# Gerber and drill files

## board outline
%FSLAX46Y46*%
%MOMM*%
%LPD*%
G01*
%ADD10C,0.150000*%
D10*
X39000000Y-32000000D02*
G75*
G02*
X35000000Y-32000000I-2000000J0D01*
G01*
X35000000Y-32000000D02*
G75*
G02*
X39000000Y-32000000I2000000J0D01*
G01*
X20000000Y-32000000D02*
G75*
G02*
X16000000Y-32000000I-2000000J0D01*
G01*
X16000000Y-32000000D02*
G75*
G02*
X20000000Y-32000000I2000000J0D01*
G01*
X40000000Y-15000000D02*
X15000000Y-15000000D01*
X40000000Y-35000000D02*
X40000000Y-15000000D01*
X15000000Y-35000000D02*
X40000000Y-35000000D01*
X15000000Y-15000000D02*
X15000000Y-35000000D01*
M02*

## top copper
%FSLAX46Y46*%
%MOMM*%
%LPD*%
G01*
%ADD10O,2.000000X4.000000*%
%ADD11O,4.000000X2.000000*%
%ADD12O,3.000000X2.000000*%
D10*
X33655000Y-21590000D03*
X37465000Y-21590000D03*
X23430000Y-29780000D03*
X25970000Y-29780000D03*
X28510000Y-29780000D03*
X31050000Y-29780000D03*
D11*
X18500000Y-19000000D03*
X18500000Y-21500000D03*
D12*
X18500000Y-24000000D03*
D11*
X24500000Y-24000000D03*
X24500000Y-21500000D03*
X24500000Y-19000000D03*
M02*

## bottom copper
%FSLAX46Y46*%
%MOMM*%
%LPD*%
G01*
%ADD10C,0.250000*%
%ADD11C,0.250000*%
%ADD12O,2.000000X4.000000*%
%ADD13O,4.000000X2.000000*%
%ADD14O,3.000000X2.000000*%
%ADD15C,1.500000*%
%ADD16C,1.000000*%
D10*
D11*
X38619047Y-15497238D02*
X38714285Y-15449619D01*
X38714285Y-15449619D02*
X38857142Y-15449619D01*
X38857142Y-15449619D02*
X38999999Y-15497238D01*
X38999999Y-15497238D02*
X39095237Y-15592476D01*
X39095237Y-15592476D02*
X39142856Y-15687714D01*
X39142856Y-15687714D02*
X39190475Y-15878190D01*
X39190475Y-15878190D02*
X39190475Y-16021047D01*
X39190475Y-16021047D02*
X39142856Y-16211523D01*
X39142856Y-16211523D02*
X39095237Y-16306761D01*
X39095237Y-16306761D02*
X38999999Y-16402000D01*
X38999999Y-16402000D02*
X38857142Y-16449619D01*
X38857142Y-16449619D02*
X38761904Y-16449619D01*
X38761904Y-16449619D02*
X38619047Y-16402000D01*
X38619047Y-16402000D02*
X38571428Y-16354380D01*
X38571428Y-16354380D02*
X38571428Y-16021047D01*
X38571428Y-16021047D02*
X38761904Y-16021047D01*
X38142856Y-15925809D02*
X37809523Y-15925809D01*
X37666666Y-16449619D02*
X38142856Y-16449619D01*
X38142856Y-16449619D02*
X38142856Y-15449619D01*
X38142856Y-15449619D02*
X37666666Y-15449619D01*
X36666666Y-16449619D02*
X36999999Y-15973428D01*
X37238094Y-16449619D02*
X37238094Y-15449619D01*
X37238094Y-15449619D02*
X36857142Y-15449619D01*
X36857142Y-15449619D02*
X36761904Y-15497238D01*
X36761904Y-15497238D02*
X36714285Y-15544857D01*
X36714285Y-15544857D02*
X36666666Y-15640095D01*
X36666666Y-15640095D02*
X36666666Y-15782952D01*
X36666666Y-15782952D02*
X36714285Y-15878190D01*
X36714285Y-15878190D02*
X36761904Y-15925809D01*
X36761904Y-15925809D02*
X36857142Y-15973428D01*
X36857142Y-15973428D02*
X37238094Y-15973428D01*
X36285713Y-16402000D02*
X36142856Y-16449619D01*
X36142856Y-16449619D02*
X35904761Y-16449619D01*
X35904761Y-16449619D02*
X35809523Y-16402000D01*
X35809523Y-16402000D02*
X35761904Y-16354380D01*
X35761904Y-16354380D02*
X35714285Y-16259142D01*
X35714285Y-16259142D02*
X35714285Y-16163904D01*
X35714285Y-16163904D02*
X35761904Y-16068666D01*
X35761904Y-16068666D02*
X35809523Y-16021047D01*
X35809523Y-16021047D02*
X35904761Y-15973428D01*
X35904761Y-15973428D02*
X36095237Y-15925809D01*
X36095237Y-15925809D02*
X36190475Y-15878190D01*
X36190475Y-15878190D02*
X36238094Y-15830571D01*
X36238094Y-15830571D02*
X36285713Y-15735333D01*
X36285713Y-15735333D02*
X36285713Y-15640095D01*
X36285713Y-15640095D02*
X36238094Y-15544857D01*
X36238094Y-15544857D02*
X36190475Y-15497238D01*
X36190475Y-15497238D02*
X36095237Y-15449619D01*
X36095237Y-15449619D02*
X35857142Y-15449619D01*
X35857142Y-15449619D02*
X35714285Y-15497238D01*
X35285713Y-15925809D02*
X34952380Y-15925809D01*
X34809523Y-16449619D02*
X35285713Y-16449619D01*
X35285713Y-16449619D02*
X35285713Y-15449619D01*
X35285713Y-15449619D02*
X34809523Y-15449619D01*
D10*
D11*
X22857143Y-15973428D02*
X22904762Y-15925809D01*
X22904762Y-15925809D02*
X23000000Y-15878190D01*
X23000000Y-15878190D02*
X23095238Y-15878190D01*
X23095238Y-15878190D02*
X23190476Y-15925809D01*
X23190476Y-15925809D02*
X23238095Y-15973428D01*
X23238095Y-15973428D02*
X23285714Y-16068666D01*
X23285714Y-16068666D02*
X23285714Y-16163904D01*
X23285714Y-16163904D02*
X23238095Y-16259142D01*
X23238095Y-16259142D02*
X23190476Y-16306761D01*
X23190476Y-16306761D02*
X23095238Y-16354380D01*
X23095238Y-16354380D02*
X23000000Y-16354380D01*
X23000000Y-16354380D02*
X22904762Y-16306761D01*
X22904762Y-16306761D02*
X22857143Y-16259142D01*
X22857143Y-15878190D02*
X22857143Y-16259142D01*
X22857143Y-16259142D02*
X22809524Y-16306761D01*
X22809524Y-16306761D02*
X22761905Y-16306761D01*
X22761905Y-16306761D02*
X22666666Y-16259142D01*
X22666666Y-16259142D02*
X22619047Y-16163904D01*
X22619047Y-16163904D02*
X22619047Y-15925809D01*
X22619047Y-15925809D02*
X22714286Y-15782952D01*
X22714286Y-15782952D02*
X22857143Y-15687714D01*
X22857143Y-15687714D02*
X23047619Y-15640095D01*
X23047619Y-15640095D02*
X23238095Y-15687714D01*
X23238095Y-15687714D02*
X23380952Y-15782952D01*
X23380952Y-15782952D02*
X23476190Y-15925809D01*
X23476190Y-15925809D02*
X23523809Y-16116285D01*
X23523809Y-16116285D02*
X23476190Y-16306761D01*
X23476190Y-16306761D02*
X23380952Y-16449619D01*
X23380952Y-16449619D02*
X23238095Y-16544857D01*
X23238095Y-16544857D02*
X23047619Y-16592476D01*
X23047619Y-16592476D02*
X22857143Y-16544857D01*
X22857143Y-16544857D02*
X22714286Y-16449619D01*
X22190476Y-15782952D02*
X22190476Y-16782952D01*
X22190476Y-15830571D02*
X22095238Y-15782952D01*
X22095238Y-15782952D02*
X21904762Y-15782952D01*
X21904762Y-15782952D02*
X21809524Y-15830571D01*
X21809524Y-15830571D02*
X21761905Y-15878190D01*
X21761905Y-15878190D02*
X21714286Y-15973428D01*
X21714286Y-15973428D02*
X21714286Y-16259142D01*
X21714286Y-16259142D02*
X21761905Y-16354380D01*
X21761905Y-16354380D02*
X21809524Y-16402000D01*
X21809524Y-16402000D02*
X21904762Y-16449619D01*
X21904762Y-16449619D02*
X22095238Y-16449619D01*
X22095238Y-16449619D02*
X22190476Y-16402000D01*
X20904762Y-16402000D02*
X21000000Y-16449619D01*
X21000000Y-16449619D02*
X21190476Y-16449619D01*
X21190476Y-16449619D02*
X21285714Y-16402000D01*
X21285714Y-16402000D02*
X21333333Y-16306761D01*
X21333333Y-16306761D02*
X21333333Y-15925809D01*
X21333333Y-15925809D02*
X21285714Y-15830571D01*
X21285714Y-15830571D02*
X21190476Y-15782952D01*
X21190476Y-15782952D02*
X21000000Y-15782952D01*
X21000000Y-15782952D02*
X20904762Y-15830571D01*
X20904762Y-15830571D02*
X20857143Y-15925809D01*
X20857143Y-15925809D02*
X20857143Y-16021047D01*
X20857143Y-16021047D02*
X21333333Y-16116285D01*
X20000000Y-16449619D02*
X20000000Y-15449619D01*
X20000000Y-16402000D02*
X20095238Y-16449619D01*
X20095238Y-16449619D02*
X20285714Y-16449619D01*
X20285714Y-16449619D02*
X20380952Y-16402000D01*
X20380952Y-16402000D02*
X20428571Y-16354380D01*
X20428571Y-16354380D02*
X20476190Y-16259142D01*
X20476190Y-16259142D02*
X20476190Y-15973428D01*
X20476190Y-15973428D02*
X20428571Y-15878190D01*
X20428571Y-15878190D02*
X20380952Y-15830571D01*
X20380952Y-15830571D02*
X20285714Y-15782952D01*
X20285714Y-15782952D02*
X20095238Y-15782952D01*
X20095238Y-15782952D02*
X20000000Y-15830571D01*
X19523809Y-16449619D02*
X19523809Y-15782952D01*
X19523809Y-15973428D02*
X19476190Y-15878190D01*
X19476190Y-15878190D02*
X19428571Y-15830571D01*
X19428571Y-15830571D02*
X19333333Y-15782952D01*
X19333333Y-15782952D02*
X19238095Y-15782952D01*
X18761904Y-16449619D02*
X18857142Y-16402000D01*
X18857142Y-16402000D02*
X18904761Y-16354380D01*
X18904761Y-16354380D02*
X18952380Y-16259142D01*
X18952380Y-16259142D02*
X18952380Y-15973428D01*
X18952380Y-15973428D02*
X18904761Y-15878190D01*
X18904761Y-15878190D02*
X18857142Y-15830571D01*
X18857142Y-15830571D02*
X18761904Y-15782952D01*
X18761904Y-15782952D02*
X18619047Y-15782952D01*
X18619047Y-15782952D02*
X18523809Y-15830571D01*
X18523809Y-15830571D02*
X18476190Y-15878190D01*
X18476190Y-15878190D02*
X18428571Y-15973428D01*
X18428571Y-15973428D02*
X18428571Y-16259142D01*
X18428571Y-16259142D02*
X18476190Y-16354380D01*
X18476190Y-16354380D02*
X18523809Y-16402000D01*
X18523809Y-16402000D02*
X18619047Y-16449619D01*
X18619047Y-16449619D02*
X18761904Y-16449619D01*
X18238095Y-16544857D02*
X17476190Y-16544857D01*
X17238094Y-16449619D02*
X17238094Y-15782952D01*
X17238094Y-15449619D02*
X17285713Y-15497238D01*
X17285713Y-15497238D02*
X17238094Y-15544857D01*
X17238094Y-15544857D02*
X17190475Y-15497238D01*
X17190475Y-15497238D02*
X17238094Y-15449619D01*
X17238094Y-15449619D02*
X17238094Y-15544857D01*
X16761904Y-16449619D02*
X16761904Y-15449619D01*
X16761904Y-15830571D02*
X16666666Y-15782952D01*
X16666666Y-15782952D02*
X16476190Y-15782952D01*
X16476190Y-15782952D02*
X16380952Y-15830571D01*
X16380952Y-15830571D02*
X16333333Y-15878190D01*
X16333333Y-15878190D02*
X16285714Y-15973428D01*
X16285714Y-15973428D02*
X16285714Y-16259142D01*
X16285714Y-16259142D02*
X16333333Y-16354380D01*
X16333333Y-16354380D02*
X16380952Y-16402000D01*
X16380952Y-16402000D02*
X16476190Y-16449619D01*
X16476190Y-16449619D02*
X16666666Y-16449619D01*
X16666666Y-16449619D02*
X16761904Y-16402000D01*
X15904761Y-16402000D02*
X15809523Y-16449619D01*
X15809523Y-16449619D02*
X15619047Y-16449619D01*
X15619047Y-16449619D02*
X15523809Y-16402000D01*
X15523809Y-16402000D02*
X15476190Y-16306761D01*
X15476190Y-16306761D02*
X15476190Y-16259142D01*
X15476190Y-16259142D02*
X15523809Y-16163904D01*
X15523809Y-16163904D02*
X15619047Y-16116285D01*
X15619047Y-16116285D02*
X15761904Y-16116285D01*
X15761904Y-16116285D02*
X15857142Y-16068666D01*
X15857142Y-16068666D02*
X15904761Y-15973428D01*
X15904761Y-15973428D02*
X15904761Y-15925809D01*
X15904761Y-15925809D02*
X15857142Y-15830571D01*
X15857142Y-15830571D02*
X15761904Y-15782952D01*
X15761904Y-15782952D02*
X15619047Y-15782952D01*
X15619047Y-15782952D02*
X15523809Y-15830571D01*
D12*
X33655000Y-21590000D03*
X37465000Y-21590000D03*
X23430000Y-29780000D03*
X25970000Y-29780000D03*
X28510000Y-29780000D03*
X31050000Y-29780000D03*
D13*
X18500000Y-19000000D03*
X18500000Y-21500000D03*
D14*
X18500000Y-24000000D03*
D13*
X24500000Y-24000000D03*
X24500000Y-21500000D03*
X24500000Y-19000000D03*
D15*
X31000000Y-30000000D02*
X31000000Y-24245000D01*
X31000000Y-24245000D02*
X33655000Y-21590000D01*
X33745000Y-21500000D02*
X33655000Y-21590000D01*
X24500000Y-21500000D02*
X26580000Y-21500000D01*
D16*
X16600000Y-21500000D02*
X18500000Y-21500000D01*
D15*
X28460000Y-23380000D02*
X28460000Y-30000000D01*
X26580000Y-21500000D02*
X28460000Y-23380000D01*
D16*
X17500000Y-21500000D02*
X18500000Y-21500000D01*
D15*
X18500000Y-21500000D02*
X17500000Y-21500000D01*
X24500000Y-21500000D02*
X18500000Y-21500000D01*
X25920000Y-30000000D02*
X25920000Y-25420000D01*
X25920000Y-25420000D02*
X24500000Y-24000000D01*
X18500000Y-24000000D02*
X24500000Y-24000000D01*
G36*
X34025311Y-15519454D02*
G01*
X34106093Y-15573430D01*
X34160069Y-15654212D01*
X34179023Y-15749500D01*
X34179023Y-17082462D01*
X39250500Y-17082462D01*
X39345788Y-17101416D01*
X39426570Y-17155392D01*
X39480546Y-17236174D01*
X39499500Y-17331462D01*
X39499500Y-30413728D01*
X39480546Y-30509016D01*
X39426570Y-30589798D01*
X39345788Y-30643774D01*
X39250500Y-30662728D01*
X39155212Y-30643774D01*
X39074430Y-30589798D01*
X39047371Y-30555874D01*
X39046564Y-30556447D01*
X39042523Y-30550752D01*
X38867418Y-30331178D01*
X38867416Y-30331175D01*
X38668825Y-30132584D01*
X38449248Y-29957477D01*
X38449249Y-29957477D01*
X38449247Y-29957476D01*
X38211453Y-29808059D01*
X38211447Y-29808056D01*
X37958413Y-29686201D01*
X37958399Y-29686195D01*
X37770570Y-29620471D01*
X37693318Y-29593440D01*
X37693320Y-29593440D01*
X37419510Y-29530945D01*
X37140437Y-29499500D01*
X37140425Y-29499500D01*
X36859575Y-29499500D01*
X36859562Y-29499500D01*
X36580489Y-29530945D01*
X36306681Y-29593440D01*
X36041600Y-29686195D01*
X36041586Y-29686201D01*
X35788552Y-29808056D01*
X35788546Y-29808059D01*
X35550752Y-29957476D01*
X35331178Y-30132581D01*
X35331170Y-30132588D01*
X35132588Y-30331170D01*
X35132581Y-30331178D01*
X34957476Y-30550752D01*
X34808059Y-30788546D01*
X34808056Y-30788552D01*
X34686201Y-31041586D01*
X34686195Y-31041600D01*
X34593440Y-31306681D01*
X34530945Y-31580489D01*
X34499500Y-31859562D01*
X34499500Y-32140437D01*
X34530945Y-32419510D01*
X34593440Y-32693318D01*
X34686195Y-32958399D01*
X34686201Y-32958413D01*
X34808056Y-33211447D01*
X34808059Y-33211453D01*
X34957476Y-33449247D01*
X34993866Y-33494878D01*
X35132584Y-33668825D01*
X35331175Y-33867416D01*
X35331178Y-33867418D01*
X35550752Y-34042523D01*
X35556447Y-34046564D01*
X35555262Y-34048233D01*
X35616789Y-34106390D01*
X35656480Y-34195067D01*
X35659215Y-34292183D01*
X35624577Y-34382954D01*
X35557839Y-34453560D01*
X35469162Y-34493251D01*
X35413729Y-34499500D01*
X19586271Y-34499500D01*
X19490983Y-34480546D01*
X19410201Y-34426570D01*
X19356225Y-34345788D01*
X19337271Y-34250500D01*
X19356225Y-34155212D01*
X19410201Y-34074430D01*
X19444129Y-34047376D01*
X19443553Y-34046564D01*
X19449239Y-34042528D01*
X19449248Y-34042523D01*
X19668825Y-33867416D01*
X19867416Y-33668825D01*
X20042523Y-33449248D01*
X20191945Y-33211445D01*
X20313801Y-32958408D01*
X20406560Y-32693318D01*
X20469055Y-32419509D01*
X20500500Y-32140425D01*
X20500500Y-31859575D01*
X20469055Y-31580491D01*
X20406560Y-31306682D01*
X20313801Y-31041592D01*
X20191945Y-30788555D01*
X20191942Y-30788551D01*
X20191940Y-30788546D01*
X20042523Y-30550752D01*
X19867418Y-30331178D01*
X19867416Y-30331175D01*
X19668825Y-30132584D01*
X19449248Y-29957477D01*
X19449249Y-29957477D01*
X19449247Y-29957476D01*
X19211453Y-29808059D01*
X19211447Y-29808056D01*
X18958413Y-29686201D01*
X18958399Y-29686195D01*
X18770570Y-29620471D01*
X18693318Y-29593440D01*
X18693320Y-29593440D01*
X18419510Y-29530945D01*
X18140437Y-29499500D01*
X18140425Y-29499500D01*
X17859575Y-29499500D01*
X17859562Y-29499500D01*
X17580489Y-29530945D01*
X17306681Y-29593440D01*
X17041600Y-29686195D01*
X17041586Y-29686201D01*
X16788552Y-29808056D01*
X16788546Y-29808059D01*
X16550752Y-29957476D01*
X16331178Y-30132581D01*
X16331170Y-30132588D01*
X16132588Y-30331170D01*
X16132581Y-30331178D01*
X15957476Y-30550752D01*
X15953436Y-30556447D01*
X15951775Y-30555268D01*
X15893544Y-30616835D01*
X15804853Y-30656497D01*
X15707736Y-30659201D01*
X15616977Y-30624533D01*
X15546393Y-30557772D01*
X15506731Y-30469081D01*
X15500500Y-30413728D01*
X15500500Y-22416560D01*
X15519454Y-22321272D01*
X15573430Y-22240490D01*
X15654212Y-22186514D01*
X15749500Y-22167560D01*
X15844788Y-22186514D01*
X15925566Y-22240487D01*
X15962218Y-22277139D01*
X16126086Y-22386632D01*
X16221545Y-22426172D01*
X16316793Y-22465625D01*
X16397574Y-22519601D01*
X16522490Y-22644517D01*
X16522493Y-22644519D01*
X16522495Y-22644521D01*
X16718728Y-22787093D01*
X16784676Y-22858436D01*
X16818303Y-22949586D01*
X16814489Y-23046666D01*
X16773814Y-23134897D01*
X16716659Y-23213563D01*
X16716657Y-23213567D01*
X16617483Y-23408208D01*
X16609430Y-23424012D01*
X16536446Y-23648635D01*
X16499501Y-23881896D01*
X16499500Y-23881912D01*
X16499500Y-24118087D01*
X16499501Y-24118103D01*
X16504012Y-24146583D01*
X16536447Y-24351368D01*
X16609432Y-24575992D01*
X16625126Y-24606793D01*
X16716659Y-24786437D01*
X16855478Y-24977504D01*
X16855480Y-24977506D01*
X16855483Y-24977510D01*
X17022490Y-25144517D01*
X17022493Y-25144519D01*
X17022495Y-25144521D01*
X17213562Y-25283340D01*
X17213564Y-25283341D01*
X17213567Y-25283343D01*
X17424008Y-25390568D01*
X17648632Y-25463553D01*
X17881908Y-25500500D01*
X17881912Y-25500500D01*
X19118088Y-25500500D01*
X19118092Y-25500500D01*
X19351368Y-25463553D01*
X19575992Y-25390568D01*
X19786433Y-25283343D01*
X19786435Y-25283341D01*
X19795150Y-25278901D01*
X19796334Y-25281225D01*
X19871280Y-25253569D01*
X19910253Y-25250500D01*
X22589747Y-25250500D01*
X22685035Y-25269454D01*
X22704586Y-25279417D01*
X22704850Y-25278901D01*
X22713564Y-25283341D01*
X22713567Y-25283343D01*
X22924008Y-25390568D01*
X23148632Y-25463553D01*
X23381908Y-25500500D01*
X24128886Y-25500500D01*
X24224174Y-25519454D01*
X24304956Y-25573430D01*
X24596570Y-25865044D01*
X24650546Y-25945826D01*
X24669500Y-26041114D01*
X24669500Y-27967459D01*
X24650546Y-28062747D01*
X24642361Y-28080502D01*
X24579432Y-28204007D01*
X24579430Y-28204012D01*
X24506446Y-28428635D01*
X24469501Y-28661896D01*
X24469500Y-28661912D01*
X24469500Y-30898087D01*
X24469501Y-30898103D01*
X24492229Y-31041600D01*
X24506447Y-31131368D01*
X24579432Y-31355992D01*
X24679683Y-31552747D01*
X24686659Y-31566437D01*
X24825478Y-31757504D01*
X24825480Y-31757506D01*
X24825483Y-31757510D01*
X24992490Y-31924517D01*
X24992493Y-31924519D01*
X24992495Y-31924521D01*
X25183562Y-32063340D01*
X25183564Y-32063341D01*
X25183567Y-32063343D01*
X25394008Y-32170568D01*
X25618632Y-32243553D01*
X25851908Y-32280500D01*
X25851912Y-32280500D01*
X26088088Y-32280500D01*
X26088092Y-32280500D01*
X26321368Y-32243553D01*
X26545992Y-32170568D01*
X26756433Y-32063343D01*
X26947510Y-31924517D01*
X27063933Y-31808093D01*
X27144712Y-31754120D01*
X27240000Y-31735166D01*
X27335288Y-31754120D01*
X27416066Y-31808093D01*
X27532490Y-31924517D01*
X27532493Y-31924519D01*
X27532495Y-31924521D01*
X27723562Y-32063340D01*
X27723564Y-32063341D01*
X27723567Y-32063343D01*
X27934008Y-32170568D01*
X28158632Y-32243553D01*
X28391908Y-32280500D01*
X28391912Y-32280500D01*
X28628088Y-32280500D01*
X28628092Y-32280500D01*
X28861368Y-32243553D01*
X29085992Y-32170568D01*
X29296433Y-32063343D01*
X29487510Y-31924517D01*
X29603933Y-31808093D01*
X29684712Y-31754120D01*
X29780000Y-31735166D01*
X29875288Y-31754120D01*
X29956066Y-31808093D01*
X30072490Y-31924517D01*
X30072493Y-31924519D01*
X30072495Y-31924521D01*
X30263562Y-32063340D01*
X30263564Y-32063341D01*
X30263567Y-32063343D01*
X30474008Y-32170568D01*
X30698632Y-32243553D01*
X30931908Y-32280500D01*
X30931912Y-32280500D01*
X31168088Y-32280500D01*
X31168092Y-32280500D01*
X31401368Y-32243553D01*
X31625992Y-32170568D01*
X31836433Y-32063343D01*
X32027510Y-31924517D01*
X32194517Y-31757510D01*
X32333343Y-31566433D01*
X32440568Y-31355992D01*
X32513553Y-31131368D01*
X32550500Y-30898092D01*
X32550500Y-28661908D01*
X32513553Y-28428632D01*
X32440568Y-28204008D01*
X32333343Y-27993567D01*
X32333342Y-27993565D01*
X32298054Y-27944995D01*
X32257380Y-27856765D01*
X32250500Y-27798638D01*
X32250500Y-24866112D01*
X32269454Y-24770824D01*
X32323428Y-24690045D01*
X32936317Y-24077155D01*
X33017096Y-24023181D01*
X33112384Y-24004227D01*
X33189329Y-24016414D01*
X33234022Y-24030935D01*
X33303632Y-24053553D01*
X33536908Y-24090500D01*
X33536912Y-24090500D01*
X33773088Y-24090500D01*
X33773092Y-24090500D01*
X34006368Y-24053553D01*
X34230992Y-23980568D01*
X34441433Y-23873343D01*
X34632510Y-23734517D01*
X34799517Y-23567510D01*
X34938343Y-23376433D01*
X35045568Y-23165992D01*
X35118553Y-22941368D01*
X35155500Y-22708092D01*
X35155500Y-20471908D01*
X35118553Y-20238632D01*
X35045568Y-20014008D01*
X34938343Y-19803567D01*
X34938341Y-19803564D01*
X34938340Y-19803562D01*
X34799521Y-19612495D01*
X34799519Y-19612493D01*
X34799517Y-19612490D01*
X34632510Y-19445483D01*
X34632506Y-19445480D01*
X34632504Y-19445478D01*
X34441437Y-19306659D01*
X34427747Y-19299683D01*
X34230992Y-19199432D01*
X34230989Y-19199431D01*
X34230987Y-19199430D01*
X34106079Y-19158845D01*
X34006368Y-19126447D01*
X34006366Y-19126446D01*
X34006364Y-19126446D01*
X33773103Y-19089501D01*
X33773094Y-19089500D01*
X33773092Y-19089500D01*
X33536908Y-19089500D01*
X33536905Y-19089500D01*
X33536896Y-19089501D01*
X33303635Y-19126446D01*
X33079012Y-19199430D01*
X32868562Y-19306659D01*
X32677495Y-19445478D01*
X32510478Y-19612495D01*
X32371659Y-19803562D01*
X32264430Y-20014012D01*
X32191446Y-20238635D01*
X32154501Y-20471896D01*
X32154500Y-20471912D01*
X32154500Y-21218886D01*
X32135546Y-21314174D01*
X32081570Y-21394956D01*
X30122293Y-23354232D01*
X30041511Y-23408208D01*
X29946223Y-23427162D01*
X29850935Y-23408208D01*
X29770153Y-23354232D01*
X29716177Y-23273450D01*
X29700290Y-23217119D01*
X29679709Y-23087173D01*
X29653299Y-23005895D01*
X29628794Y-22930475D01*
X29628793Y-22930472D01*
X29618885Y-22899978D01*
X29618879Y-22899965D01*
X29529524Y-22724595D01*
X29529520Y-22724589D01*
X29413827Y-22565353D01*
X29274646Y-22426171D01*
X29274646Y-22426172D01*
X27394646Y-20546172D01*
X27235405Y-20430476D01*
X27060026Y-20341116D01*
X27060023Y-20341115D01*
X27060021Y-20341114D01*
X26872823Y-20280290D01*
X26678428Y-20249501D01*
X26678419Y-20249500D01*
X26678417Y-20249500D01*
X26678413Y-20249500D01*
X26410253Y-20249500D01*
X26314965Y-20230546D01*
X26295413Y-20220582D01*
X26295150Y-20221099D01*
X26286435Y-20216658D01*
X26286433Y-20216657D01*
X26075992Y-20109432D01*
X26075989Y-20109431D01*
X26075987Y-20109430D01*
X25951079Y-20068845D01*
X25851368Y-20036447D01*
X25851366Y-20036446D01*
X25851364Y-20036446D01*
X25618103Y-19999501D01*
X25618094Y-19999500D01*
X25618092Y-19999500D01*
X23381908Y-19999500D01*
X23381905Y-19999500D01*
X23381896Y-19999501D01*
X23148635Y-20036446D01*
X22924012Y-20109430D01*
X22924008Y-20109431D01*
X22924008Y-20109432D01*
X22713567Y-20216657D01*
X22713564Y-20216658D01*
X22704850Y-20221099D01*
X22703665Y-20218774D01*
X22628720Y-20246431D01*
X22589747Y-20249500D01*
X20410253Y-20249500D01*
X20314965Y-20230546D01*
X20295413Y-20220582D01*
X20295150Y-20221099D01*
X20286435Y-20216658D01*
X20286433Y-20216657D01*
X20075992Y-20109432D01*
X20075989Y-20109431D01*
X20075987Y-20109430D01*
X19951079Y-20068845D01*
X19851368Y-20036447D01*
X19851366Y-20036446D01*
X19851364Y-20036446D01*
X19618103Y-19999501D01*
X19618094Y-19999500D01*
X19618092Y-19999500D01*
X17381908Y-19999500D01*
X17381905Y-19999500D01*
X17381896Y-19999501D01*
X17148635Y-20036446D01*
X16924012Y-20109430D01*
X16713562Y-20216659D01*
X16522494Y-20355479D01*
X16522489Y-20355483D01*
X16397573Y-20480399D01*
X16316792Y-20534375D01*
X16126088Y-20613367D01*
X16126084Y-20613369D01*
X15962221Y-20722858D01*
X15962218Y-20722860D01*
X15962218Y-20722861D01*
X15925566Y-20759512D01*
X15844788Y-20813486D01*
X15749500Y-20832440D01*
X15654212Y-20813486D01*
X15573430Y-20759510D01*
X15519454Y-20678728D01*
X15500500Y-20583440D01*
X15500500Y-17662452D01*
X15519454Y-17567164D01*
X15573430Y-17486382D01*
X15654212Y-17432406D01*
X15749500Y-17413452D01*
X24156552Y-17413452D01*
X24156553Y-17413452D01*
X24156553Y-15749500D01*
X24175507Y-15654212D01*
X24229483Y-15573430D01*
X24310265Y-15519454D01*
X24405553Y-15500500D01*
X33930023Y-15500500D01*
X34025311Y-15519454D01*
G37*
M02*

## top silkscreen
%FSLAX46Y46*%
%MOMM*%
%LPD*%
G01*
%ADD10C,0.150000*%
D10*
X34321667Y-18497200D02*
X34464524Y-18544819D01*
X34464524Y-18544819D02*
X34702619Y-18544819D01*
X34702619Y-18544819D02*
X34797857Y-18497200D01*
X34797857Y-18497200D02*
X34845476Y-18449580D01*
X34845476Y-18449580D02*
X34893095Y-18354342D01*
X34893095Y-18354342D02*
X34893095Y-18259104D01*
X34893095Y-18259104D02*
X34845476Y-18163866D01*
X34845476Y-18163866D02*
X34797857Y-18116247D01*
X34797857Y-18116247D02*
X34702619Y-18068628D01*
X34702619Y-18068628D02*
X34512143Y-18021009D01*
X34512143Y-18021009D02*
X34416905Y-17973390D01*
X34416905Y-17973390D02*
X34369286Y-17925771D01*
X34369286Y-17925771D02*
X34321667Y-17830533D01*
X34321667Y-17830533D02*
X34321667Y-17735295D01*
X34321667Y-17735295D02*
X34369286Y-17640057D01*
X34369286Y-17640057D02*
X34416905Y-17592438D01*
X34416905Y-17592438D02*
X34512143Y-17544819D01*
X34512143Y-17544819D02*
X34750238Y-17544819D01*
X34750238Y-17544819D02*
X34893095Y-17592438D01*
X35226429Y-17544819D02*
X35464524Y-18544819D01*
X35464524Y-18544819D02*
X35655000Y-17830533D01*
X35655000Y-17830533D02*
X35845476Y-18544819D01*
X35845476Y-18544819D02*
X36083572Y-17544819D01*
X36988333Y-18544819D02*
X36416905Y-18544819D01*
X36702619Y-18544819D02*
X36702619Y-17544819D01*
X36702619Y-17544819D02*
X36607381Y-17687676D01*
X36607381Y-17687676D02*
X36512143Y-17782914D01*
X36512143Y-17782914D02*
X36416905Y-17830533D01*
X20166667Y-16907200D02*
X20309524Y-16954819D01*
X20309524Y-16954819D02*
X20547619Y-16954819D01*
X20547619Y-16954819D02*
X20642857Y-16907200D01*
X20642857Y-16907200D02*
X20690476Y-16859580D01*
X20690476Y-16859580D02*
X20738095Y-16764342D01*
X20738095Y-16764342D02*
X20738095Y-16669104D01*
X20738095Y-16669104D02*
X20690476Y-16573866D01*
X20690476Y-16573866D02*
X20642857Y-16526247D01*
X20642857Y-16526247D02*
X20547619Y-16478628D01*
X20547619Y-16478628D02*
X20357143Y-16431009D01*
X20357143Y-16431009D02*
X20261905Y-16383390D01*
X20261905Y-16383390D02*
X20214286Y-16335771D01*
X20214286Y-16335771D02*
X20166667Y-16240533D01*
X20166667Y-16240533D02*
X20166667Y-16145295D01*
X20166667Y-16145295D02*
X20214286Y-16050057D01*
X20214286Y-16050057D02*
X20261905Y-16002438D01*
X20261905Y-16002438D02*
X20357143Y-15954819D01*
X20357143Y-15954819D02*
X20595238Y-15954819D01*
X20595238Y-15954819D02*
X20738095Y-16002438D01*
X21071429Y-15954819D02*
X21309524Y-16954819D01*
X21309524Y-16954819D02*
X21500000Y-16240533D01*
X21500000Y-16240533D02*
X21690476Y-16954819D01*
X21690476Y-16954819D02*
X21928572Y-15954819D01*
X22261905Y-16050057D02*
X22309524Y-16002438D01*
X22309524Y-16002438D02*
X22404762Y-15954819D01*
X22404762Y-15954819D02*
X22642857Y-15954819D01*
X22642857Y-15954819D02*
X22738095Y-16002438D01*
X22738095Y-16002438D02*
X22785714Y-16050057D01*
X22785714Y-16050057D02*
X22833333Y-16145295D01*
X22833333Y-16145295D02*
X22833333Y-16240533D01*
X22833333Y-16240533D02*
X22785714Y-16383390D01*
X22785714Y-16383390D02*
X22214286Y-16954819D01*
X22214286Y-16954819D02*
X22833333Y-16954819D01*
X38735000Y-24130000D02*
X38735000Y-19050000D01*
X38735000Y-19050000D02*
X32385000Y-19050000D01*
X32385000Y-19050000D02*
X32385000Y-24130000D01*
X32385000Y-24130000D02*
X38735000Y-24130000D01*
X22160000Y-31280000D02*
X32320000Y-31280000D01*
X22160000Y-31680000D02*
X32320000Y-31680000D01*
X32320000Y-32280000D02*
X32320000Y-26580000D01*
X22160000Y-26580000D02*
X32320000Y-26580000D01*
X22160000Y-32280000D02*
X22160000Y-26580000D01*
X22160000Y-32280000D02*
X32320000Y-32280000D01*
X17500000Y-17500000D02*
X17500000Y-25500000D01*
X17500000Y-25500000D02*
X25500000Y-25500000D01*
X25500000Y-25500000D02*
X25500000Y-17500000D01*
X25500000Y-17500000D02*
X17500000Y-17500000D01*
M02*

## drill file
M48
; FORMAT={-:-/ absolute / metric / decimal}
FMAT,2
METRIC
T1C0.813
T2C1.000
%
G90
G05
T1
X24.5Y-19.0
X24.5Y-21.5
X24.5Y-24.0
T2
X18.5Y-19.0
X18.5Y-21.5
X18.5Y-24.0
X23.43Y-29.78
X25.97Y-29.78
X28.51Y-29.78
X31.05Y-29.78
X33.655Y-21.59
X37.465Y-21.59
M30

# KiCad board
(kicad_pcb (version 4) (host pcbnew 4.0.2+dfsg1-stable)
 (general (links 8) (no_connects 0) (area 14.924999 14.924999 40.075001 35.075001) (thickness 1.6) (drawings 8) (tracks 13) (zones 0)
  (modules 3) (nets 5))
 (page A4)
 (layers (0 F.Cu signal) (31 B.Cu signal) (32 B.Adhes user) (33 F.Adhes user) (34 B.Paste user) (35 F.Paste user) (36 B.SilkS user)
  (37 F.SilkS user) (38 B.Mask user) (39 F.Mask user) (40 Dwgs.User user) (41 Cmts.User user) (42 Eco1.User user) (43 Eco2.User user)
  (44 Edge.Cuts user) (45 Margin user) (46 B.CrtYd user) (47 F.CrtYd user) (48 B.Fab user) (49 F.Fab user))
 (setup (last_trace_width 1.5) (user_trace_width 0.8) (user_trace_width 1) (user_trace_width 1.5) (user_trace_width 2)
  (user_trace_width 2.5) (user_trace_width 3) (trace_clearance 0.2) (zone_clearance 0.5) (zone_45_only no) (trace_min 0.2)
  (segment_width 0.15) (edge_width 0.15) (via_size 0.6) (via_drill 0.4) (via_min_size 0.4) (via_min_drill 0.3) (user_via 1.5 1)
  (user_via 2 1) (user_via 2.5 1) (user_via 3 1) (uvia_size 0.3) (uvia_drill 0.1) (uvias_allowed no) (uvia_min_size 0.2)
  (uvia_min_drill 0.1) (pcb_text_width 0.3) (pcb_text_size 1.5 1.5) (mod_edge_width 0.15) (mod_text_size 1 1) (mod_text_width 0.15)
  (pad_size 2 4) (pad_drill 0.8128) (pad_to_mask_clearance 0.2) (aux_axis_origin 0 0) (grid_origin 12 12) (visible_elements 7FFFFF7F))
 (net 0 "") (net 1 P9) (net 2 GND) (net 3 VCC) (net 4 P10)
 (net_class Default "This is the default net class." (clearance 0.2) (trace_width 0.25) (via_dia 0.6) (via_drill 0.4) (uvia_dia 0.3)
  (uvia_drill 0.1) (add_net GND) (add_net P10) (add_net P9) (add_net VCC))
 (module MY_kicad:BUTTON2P (layer F.Cu) (at 33.655 21.59)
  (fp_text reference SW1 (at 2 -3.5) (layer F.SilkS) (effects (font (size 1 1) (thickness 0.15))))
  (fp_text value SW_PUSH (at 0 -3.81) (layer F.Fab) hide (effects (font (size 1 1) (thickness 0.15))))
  (fp_line (start 5.08 2.54) (end 5.08 -2.54) (layer F.SilkS) (width 0.15))
  (fp_line (start 5.08 -2.54) (end -1.27 -2.54) (layer F.SilkS) (width 0.15))
  (fp_line (start -1.27 -2.54) (end -1.27 2.54) (layer F.SilkS) (width 0.15))
  (fp_line (start -1.27 2.54) (end 5.08 2.54) (layer F.SilkS) (width 0.15))
  (pad 1 thru_hole oval (at 0 0) (size 2 4) (drill 1) (layers *.Cu *.Mask) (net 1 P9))
  (pad 2 thru_hole oval (at 3.81 0) (size 2 4) (drill 1) (layers *.Cu *.Mask) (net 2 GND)))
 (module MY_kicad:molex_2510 (layer F.Cu) (at 23.43 29.78)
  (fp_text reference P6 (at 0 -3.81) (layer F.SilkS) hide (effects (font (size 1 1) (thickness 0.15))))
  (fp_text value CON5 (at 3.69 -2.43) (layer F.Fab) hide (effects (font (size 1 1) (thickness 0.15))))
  (fp_line (start -1.27 1.5) (end 8.89 1.5) (layer F.SilkS) (width 0.15))
  (fp_line (start -1.27 1.9) (end 8.89 1.9) (layer F.SilkS) (width 0.15))
  (fp_line (start 8.89 2.5) (end 8.89 -3.2) (layer F.SilkS) (width 0.15))
  (fp_line (start -1.27 -3.2) (end 8.89 -3.2) (layer F.SilkS) (width 0.15))
  (fp_line (start -1.27 2.5) (end -1.27 -3.2) (layer F.SilkS) (width 0.15))
  (fp_line (start -1.27 2.5) (end 8.89 2.5) (layer F.SilkS) (width 0.15))
  (pad 1 thru_hole oval (at 0 0) (size 2 4) (drill 1) (layers *.Cu *.Mask) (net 2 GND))
  (pad 2 thru_hole oval (at 2.54 0) (size 2 4) (drill 1) (layers *.Cu *.Mask) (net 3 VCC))
  (pad 3 thru_hole oval (at 5.08 0) (size 2 4) (drill 1) (layers *.Cu *.Mask) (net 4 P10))
  (pad 4 thru_hole oval (at 7.62 0) (size 2 4) (drill 1) (layers *.Cu *.Mask) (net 1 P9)))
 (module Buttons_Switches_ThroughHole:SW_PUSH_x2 (layer F.Cu) (at 18.5 19 270)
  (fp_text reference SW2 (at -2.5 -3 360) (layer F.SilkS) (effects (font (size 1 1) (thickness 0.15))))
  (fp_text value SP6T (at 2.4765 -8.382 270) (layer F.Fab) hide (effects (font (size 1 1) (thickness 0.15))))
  (fp_line (start -1.5 1) (end 6.5 1) (layer F.SilkS) (width 0.15))
  (fp_line (start 6.5 1) (end 6.5 -7) (layer F.SilkS) (width 0.15))
  (fp_line (start 6.5 -7) (end -1.5 -7) (layer F.SilkS) (width 0.15))
  (fp_line (start -1.5 -7) (end -1.5 1) (layer F.SilkS) (width 0.15))
  (pad 1 thru_hole oval (at 0 0 270) (size 2 4) (drill 1) (layers *.Cu *.Mask) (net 2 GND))
  (pad 2 thru_hole oval (at 2.5 0 270) (size 2 4) (drill 1) (layers *.Cu B.Mask) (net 4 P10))
  (pad 3 thru_hole oval (at 5 0 270) (size 2 3) (drill 1) (layers *.Cu *.Mask) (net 3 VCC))
  (pad 4 thru_hole oval (at 5 -6 270) (size 2 4) (drill 0.8128) (layers *.Cu *.Mask) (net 3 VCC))
  (pad 5 thru_hole oval (at 2.5 -6 270) (size 2 4) (drill 0.8128) (layers *.Cu *.Mask) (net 4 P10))
  (pad 6 thru_hole oval (at 0 -6 270) (size 2 4) (drill 0.8128) (layers *.Cu *.Mask) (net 2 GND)))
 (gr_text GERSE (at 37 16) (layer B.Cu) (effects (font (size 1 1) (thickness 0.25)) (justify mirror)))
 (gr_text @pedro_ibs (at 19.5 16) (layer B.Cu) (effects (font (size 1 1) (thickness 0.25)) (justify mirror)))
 (gr_circle (center 37 32) (end 39 32) (layer Edge.Cuts) (width 0.15))
 (gr_circle (center 18 32) (end 20 32) (layer Edge.Cuts) (width 0.15))
 (gr_line (start 40 15) (end 15 15) (angle 90) (layer Edge.Cuts) (width 0.15))
 (gr_line (start 40 35) (end 40 15) (angle 90) (layer Edge.Cuts) (width 0.15))
 (gr_line (start 15 35) (end 40 35) (angle 90) (layer Edge.Cuts) (width 0.15))
 (gr_line (start 15 15) (end 15 35) (angle 90) (layer Edge.Cuts) (width 0.15))
 (segment (start 31 30) (end 31 24.245) (width 1.5) (layer B.Cu) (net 1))
 (segment (start 31 24.245) (end 33.655 21.59) (width 1.5) (layer B.Cu) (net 1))
 (segment (start 33.745 21.5) (end 33.655 21.59) (width 1.5) (layer B.Cu) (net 1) (status 30))
 (segment (start 24.5 21.5) (end 26.58 21.5) (width 1.5) (layer B.Cu) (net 4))
 (segment (start 16.6 21.5) (end 18.5 21.5) (width 1) (layer B.Cu) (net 4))
 (segment (start 28.46 23.38) (end 28.46 30) (width 1.5) (layer B.Cu) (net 4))
 (segment (start 26.58 21.5) (end 28.46 23.38) (width 1.5) (layer B.Cu) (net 4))
 (segment (start 17.5 21.5) (end 18.5 21.5) (width 1) (layer B.Cu) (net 4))
 (segment (start 18.5 21.5) (end 17.5 21.5) (width 1.5) (layer B.Cu) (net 4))
 (segment (start 24.5 21.5) (end 18.5 21.5) (width 1.5) (layer B.Cu) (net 4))
 (segment (start 25.92 30) (end 25.92 25.42) (width 1.5) (layer B.Cu) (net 3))
 (segment (start 25.92 25.42) (end 24.5 24) (width 1.5) (layer B.Cu) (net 3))
 (segment (start 18.5 24) (end 24.5 24) (width 1.5) (layer B.Cu) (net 3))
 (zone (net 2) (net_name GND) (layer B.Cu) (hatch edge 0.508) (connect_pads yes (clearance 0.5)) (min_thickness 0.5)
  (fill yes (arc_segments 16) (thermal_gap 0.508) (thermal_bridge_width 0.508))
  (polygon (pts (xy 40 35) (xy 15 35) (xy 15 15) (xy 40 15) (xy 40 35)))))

